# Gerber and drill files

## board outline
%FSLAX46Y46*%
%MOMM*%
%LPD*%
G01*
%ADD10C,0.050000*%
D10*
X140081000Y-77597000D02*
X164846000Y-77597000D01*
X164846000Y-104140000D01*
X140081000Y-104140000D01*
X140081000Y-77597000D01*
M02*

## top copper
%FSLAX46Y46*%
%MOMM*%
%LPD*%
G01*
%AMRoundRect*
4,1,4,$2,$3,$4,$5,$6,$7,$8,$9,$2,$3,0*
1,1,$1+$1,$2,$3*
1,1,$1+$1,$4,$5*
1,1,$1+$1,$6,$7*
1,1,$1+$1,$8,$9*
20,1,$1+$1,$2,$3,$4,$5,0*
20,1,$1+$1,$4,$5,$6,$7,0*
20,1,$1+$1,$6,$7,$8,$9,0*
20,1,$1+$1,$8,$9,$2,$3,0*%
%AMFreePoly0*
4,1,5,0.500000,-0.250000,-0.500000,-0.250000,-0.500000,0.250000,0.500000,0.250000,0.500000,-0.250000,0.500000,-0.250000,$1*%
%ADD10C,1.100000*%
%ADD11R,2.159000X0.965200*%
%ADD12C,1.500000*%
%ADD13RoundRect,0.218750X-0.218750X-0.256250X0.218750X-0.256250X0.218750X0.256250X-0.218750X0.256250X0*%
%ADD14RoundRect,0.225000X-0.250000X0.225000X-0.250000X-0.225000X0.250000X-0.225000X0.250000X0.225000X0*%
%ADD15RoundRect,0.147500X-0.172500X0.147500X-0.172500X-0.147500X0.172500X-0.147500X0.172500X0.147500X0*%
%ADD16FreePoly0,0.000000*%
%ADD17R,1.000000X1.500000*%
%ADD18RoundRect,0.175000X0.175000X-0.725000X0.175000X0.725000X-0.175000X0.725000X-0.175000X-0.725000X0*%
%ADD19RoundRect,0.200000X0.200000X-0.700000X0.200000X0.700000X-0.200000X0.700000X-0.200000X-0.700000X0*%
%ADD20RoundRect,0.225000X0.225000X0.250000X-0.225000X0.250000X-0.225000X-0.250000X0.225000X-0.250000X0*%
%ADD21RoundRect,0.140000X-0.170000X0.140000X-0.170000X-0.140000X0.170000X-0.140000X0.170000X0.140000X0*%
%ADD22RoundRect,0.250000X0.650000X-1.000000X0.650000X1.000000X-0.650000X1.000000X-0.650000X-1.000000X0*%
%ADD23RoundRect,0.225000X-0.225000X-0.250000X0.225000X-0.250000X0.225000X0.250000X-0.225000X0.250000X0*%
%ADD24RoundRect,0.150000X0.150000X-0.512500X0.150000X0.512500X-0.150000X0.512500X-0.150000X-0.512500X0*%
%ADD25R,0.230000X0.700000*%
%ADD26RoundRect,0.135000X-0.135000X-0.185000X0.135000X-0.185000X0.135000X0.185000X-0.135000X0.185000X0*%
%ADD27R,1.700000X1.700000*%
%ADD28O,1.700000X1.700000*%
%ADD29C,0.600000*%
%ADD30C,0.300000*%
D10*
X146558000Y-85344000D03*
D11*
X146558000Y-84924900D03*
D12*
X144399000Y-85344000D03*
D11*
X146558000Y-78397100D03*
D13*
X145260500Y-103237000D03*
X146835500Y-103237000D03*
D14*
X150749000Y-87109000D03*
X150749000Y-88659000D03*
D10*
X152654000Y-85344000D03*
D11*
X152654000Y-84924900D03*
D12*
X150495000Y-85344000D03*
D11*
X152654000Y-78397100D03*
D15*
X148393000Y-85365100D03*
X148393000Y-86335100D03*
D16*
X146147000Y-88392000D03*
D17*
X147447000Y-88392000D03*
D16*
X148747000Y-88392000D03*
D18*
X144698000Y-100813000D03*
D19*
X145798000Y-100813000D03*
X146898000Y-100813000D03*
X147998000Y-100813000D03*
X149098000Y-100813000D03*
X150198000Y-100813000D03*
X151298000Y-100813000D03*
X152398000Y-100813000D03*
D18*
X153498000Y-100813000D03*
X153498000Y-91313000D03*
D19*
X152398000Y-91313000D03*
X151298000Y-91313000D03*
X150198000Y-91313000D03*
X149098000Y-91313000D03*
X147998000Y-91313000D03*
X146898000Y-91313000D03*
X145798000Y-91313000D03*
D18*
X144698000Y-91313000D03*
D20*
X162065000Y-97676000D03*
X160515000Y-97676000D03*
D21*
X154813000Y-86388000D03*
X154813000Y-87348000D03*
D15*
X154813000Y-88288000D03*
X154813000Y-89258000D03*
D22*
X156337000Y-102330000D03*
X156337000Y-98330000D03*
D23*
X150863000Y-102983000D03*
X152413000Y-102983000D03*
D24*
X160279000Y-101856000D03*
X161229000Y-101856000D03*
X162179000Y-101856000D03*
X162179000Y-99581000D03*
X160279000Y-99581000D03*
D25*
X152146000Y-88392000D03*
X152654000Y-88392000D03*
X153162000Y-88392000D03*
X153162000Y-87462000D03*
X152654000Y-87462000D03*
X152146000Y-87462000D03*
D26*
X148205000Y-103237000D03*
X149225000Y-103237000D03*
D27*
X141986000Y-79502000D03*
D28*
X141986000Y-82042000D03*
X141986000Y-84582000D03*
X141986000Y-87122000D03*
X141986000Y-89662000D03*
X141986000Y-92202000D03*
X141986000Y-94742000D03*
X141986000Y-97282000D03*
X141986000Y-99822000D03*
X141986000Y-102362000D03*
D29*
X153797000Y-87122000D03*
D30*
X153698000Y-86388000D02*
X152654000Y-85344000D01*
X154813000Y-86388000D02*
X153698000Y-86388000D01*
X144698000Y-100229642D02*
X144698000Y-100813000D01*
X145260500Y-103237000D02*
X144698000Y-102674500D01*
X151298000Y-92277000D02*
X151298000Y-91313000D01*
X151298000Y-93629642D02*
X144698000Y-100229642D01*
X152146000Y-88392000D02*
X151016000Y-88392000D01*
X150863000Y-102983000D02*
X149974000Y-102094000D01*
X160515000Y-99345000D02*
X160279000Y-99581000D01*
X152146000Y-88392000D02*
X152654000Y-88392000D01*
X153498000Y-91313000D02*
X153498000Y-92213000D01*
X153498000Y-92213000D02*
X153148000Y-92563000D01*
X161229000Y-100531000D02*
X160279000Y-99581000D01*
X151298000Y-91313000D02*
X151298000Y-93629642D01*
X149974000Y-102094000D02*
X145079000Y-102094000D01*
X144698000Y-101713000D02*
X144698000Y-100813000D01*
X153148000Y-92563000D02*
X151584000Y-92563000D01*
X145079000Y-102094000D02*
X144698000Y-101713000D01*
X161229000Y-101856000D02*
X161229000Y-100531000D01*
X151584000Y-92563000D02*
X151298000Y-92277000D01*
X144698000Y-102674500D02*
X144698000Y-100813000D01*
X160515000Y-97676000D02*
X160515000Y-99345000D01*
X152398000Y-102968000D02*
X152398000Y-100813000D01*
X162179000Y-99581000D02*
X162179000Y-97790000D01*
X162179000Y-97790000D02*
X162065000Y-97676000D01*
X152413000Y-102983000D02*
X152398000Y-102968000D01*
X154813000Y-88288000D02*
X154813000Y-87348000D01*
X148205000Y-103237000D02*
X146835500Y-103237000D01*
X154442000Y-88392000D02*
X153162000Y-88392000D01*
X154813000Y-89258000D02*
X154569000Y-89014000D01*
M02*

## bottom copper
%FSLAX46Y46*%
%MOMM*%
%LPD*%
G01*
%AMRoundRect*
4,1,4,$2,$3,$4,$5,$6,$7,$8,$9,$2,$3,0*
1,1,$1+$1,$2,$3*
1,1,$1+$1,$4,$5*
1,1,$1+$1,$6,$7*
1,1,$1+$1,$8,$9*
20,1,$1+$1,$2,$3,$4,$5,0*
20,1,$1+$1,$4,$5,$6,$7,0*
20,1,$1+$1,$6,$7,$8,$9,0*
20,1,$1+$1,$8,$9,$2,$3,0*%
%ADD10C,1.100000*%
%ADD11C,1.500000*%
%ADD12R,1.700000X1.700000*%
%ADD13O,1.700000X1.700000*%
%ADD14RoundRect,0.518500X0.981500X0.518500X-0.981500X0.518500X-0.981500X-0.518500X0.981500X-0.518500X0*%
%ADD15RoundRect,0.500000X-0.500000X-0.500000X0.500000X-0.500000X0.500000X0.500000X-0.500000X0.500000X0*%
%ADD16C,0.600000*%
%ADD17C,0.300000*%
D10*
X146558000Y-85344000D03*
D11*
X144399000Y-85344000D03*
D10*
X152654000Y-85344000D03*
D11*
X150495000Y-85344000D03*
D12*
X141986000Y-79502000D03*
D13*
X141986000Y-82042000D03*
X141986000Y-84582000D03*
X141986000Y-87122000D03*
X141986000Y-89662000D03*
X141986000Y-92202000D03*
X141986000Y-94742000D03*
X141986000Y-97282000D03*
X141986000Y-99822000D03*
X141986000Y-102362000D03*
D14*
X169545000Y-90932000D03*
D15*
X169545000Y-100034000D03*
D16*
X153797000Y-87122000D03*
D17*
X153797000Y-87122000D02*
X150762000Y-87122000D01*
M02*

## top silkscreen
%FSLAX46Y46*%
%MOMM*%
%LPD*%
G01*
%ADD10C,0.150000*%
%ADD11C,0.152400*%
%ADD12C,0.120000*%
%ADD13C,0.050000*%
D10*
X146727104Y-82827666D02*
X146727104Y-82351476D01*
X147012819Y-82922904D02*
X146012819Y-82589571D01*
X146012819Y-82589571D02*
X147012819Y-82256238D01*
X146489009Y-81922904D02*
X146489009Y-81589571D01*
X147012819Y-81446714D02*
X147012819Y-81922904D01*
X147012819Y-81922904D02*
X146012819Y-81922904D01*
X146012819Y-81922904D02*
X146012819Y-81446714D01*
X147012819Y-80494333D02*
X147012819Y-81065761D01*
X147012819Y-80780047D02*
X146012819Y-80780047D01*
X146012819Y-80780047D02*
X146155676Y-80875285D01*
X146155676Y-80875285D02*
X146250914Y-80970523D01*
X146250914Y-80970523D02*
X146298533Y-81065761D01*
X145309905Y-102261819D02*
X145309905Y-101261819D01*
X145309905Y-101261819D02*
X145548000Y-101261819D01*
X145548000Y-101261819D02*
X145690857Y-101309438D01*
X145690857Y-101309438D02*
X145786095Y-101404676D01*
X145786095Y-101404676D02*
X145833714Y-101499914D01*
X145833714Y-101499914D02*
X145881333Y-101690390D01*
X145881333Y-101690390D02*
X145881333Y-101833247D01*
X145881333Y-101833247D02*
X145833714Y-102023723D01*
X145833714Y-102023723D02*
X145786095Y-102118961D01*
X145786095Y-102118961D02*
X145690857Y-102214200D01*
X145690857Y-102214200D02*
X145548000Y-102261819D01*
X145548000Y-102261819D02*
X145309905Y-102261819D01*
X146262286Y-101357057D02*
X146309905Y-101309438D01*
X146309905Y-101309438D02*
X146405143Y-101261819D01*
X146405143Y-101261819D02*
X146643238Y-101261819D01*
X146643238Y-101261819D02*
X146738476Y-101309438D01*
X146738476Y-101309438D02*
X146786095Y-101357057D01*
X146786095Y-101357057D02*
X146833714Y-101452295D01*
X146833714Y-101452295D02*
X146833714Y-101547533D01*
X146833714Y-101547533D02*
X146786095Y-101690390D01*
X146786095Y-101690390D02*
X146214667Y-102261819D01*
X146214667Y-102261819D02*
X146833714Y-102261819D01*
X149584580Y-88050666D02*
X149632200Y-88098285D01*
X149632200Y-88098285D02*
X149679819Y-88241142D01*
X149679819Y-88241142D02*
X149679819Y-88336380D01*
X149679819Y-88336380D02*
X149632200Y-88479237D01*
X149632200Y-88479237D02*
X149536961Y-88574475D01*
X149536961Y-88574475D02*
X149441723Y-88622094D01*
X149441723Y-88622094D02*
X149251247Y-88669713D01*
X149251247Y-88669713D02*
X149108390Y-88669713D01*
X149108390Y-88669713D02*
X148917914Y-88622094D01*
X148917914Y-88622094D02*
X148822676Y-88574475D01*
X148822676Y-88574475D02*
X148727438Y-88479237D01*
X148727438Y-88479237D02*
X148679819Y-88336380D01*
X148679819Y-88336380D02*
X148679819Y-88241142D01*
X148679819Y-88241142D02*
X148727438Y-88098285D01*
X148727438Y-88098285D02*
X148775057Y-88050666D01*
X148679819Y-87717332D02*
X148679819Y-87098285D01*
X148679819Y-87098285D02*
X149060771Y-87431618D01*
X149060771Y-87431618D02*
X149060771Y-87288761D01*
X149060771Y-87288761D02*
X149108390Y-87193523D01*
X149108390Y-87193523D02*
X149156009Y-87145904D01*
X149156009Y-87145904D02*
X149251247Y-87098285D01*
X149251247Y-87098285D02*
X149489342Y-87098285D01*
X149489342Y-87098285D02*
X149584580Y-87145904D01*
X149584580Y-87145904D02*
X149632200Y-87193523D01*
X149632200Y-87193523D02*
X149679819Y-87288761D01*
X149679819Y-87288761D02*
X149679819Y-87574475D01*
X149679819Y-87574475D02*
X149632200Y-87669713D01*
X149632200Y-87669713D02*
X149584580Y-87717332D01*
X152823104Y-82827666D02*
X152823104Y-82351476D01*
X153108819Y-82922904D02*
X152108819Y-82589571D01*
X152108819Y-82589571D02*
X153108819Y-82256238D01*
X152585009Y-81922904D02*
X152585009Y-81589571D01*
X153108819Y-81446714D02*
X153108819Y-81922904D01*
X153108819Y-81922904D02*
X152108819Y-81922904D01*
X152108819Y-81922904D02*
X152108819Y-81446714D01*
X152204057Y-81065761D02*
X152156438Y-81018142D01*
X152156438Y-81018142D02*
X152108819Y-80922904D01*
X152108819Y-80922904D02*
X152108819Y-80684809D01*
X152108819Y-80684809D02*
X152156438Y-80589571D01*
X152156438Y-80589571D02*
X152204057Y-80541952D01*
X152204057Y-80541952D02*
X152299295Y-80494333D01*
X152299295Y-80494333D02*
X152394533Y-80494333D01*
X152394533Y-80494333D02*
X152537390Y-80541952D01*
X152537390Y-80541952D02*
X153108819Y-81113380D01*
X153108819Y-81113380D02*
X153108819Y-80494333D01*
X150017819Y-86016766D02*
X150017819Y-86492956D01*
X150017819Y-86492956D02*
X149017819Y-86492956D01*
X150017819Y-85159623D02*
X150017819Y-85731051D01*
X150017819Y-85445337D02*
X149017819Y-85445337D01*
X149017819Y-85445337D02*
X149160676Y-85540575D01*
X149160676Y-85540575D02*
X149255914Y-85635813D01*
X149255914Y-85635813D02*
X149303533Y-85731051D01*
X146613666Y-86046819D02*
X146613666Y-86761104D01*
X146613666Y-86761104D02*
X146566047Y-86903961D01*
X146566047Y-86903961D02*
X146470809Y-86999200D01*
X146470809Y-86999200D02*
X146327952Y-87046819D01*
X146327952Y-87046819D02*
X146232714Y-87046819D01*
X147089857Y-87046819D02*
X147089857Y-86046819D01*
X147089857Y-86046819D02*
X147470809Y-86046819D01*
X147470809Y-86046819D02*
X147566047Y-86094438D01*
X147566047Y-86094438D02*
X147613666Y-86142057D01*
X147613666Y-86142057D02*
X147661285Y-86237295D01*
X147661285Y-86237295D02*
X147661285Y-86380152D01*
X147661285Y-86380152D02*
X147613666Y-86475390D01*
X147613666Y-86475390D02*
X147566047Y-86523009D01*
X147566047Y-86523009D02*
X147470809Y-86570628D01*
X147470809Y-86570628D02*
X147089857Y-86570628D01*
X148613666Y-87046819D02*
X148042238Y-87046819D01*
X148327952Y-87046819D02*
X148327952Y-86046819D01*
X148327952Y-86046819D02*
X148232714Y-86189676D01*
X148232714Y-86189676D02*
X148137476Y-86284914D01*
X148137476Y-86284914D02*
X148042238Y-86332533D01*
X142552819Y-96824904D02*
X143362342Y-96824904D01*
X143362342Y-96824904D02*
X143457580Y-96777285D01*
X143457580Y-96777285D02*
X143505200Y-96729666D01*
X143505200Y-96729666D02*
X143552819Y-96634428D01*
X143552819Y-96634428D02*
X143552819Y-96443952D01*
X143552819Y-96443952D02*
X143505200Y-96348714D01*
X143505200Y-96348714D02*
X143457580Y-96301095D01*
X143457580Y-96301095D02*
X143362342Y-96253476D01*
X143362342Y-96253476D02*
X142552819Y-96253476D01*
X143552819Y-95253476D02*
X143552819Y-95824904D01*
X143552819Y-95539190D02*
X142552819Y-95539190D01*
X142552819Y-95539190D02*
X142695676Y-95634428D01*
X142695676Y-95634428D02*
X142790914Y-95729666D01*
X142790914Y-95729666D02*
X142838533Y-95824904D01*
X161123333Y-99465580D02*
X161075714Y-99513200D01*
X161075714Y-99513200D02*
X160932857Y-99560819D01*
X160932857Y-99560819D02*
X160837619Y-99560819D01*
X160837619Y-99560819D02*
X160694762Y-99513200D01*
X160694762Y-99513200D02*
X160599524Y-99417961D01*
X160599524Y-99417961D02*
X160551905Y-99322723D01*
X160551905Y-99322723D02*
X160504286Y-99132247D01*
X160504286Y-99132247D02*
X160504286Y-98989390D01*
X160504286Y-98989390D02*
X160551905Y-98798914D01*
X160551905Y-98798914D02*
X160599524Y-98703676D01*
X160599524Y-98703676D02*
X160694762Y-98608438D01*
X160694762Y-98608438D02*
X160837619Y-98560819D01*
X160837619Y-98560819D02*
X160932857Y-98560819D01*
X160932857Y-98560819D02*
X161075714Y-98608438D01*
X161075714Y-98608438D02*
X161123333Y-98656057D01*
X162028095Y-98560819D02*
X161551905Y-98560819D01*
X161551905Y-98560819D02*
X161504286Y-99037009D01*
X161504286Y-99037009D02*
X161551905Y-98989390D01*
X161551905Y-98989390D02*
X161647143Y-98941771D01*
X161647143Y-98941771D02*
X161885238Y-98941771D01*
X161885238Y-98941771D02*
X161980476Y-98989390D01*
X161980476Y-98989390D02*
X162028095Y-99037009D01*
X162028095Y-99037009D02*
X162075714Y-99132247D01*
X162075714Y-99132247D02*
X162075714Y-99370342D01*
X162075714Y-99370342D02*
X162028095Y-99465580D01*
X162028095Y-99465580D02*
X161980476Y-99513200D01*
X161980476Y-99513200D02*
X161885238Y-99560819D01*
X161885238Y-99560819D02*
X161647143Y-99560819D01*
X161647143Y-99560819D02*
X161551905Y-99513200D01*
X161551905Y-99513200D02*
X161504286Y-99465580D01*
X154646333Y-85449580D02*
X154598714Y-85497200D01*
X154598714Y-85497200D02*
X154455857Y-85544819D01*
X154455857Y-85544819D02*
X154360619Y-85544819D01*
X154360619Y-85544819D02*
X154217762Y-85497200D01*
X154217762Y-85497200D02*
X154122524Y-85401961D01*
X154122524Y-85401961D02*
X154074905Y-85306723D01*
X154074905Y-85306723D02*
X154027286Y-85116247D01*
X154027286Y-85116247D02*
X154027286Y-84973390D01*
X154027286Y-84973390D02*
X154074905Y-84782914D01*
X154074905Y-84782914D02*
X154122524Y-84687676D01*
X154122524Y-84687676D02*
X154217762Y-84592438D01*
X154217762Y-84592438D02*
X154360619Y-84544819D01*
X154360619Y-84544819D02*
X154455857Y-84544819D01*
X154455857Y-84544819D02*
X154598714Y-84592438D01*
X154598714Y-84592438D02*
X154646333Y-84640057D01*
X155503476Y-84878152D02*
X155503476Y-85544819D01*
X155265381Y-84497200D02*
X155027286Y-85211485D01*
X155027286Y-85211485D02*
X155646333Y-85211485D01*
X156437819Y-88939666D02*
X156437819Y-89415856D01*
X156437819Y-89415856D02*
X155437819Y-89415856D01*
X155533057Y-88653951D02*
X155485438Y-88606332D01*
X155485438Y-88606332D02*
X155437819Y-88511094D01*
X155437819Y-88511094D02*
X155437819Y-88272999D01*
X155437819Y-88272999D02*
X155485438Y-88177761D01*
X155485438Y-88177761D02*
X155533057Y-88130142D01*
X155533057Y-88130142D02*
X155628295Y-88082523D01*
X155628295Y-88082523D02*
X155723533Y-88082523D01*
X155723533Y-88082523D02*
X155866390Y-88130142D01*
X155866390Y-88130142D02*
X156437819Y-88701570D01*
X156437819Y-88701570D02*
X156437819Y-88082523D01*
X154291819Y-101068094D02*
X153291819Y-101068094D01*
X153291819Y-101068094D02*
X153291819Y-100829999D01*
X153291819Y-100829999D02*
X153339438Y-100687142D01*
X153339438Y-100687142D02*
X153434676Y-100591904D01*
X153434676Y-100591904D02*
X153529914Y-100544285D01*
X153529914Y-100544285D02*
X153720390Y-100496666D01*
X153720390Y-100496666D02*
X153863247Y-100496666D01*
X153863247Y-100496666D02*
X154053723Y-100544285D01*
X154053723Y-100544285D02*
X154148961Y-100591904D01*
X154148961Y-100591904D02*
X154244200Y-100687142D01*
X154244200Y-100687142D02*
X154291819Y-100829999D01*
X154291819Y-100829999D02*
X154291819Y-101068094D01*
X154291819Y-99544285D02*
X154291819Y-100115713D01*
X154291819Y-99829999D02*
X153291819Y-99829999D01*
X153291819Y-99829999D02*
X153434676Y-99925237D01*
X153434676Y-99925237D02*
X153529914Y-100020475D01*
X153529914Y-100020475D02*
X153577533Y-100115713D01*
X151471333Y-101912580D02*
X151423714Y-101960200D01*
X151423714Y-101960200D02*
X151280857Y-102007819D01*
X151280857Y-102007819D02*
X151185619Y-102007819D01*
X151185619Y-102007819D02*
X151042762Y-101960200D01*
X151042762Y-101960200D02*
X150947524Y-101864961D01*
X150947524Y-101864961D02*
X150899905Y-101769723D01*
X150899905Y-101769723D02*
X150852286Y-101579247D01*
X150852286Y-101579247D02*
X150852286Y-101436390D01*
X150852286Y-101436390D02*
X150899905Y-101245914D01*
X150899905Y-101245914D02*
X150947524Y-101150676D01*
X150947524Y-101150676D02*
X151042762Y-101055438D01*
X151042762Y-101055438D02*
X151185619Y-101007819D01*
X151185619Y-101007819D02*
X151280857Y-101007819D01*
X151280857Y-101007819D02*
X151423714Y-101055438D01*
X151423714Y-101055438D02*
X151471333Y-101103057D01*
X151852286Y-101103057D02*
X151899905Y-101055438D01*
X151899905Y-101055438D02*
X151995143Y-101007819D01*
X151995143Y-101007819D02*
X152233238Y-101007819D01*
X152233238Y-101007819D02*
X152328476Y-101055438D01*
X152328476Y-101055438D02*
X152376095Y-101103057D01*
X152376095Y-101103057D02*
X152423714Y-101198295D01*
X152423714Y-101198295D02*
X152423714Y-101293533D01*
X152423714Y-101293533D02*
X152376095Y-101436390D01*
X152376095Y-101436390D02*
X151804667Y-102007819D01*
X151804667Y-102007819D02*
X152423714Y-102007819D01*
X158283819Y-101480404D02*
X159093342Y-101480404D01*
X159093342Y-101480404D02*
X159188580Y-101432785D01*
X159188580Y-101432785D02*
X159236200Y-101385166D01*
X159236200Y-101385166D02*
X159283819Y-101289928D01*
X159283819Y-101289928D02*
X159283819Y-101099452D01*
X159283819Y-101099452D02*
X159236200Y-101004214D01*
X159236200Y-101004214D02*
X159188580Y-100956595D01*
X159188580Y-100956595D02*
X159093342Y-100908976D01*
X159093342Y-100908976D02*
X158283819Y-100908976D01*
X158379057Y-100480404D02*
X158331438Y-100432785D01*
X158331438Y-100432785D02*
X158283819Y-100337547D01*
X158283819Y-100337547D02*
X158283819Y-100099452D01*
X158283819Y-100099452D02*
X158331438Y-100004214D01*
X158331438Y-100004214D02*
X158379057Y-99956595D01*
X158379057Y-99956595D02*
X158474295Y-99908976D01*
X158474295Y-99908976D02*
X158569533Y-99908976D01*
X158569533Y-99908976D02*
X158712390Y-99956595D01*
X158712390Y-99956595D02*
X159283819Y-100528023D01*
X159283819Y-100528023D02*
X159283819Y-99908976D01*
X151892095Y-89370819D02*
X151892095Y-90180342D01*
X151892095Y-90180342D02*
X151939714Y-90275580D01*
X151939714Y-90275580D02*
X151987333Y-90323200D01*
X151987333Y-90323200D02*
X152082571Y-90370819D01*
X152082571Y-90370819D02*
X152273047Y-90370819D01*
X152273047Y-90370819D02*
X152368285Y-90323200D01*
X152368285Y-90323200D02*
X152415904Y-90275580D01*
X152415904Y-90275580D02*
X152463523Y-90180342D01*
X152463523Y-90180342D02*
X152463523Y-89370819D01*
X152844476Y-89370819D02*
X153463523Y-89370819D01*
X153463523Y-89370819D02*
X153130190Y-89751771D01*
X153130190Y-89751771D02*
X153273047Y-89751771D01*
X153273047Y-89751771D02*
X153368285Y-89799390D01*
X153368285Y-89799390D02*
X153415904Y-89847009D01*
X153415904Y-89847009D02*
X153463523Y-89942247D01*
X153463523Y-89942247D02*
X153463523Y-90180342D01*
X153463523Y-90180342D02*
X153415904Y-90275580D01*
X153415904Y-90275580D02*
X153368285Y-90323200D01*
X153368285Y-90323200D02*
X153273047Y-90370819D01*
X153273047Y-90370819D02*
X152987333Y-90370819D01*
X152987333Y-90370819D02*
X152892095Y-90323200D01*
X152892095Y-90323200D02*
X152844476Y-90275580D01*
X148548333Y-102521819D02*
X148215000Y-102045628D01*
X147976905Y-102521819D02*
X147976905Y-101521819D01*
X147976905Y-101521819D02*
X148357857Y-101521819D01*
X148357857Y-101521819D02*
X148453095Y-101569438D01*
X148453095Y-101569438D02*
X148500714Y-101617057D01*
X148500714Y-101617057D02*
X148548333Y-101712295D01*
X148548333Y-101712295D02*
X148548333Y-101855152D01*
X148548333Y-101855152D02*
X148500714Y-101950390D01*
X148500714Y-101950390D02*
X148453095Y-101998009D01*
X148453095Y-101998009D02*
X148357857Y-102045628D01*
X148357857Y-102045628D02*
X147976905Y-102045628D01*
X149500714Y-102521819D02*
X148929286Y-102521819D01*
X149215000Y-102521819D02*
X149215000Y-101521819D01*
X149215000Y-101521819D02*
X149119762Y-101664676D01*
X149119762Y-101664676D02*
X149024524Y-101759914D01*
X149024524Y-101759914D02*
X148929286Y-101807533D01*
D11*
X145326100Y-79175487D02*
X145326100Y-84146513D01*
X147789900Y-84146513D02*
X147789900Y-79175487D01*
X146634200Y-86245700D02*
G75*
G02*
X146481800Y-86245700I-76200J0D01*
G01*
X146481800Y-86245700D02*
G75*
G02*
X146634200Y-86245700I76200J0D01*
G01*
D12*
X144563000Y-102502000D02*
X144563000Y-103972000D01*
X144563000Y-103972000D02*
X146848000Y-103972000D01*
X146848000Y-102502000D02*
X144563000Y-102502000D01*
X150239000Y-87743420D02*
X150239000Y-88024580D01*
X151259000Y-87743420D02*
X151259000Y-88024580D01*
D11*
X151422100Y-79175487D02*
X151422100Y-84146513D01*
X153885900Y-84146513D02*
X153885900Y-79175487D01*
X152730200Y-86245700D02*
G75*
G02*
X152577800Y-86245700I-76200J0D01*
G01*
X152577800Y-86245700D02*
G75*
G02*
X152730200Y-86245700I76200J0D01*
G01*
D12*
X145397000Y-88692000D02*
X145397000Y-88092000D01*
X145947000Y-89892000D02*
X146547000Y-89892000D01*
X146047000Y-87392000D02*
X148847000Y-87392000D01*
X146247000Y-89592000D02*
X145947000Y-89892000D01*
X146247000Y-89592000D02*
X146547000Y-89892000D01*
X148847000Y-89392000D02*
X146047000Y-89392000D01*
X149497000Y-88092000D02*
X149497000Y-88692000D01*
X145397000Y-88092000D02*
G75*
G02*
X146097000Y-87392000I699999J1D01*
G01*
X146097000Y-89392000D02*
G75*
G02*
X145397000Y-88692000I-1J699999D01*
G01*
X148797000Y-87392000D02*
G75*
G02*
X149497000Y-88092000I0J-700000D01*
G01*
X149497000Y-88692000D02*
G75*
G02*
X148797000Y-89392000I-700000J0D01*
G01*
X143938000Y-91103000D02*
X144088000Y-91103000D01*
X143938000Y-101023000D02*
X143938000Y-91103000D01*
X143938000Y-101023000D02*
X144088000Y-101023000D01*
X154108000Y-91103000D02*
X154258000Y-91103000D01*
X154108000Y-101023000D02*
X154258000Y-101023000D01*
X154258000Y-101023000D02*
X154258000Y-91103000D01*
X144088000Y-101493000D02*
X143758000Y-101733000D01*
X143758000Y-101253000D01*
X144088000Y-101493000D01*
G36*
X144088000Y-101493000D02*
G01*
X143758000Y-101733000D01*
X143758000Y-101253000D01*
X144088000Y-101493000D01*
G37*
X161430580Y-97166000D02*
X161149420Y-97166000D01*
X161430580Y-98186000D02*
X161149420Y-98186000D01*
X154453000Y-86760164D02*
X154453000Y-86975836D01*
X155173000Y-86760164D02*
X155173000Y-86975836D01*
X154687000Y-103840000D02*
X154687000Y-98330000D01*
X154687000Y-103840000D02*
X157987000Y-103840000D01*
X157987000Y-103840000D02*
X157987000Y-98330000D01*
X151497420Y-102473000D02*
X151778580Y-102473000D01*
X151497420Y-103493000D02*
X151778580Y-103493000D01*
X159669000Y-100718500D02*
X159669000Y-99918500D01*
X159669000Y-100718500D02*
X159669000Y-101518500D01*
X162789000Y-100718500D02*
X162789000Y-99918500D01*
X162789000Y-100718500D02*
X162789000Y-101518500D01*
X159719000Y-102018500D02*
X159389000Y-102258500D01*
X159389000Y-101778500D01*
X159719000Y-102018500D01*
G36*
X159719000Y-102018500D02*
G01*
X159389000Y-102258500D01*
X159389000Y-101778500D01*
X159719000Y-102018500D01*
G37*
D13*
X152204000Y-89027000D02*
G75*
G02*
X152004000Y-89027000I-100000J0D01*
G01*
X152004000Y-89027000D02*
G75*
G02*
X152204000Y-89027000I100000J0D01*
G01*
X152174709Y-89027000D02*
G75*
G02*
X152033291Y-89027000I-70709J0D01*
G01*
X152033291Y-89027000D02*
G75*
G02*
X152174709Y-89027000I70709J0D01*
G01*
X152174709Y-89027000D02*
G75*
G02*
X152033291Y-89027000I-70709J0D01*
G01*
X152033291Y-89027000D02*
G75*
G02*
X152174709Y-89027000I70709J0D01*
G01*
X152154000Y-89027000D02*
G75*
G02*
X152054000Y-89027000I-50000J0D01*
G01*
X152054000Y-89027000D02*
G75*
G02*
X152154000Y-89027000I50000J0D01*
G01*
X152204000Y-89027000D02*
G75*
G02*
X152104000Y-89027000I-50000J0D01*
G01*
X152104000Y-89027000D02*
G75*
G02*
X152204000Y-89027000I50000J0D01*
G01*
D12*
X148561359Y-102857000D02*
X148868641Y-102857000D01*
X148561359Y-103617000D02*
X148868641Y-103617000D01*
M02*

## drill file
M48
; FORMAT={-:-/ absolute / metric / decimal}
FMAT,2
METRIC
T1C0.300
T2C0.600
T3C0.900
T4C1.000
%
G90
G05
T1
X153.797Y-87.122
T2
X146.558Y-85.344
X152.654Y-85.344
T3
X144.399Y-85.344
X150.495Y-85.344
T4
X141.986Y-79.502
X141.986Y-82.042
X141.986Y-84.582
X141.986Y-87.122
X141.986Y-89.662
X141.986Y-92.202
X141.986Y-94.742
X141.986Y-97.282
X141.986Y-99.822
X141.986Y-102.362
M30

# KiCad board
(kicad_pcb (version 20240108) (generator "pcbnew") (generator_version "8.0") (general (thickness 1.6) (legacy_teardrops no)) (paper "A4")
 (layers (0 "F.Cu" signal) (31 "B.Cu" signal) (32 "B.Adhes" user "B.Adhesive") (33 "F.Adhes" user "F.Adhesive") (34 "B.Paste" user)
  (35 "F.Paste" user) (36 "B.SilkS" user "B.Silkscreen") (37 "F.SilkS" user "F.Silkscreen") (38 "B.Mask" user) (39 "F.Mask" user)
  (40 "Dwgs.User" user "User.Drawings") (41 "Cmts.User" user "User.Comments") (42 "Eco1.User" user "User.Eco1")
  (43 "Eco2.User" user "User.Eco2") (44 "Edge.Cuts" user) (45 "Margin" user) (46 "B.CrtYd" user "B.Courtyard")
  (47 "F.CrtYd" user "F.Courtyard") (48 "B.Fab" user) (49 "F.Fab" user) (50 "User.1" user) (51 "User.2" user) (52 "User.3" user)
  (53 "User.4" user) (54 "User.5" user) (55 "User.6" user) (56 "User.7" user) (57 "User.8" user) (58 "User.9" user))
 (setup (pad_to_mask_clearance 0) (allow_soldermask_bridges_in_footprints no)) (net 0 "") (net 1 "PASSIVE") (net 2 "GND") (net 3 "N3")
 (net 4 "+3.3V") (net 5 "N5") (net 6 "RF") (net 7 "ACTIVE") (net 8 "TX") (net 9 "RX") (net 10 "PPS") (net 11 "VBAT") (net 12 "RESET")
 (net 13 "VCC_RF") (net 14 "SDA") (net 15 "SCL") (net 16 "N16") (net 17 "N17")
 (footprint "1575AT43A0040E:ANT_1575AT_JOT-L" (layer "F.Cu") (at 146.558 81.661 90)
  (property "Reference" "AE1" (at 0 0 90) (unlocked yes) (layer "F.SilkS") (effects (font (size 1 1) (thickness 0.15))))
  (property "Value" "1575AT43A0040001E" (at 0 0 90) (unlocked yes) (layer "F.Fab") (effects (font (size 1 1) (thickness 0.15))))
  (fp_line (start 2.485513 -1.2319) (end -2.485513 -1.2319) (stroke (width 0.1524) (type solid)) (layer "F.SilkS"))
  (fp_line (start -2.485513 1.2319) (end 2.485513 1.2319) (stroke (width 0.1524) (type solid)) (layer "F.SilkS"))
  (fp_circle (center -4.5847 0) (end -4.5085 0) (stroke (width 0.1524) (type solid)) (fill none) (layer "F.SilkS"))
  (pad "1" thru_hole circle (at -3.683 0 90) (size 1.1 1.1) (drill 0.6) (layers "*.Cu" "*.Mask") (remove_unused_layers no) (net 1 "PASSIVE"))
  (pad "1" smd rect (at -3.2639 0 90) (size 0.9652 2.159) (layers "F.Cu" "F.Paste" "F.Mask") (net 1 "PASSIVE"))
  (pad "2" thru_hole circle (at -3.683 -2.159 90) (size 1.5 1.5) (drill 0.9) (layers "*.Cu" "*.Mask") (remove_unused_layers no)
   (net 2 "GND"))
  (pad "3" smd rect (at 3.2639 0 90) (size 0.9652 2.159) (layers "F.Cu" "F.Paste" "F.Mask"))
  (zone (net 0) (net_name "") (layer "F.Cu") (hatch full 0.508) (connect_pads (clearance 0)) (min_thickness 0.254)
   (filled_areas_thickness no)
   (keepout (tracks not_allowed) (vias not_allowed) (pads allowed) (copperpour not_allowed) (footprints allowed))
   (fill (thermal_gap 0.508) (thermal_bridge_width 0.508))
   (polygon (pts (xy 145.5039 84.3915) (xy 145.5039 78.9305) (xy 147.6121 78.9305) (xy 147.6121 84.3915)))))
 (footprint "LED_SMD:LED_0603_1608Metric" (layer "F.Cu") (at 146.048 103.237)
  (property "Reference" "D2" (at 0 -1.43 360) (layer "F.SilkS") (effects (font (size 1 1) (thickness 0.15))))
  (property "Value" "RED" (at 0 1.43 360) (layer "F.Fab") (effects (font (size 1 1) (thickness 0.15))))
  (fp_line (start -1.485 -0.735) (end -1.485 0.735) (stroke (width 0.12) (type solid)) (layer "F.SilkS"))
  (fp_line (start -1.485 0.735) (end 0.8 0.735) (stroke (width 0.12) (type solid)) (layer "F.SilkS"))
  (fp_line (start 0.8 -0.735) (end -1.485 -0.735) (stroke (width 0.12) (type solid)) (layer "F.SilkS"))
  (pad "1" smd roundrect (at -0.7875 0) (size 0.875 0.95) (layers "F.Cu" "F.Paste" "F.Mask") (roundrect_rratio 0.25) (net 2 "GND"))
  (pad "2" smd roundrect (at 0.7875 0) (size 0.875 0.95) (layers "F.Cu" "F.Paste" "F.Mask") (roundrect_rratio 0.25) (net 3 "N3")))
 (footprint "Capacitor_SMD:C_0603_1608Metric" (layer "F.Cu") (at 150.749 87.884 -90)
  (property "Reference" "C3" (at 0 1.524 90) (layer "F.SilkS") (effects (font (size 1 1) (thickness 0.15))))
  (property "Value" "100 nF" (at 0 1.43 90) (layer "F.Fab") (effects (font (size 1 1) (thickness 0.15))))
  (fp_line (start -0.14058 0.51) (end 0.14058 0.51) (stroke (width 0.12) (type solid)) (layer "F.SilkS"))
  (fp_line (start -0.14058 -0.51) (end 0.14058 -0.51) (stroke (width 0.12) (type solid)) (layer "F.SilkS"))
  (pad "1" smd roundrect (at -0.775 0 270) (size 0.9 0.95) (layers "F.Cu" "F.Paste" "F.Mask") (roundrect_rratio 0.25) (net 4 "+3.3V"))
  (pad "2" smd roundrect (at 0.775 0 270) (size 0.9 0.95) (layers "F.Cu" "F.Paste" "F.Mask") (roundrect_rratio 0.25) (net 2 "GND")))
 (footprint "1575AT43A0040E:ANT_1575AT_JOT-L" (layer "F.Cu") (at 152.654 81.661 90)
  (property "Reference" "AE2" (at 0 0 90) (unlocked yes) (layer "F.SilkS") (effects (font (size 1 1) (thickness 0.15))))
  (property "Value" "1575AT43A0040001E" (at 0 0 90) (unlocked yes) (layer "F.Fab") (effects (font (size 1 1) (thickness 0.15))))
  (fp_line (start 2.485513 -1.2319) (end -2.485513 -1.2319) (stroke (width 0.1524) (type solid)) (layer "F.SilkS"))
  (fp_line (start -2.485513 1.2319) (end 2.485513 1.2319) (stroke (width 0.1524) (type solid)) (layer "F.SilkS"))
  (fp_circle (center -4.5847 0) (end -4.5085 0) (stroke (width 0.1524) (type solid)) (fill none) (layer "F.SilkS"))
  (pad "1" thru_hole circle (at -3.683 0 90) (size 1.1 1.1) (drill 0.6) (layers "*.Cu" "*.Mask") (remove_unused_layers no) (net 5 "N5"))
  (pad "1" smd rect (at -3.2639 0 90) (size 0.9652 2.159) (layers "F.Cu" "F.Paste" "F.Mask") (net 5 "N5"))
  (pad "2" thru_hole circle (at -3.683 -2.159 90) (size 1.5 1.5) (drill 0.9) (layers "*.Cu" "*.Mask") (remove_unused_layers no)
   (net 2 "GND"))
  (pad "3" smd rect (at 3.2639 0 90) (size 0.9652 2.159) (layers "F.Cu" "F.Paste" "F.Mask"))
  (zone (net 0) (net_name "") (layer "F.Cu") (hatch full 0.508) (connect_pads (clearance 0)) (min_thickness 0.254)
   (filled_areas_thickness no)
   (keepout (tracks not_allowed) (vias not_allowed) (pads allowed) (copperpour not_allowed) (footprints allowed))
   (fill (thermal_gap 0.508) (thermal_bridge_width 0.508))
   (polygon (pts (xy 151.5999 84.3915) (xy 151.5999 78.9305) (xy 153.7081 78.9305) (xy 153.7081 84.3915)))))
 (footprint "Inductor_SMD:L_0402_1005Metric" (layer "F.Cu") (at 148.393 85.8501 -90)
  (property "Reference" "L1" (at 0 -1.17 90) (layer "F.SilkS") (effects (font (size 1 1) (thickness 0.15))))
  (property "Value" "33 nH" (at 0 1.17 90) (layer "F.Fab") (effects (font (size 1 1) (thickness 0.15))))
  (pad "1" smd roundrect (at -0.485 0 270) (size 0.59 0.64) (layers "F.Cu" "F.Paste" "F.Mask") (roundrect_rratio 0.25) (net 1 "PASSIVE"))
  (pad "2" smd roundrect (at 0.485 0 270) (size 0.59 0.64) (layers "F.Cu" "F.Paste" "F.Mask") (roundrect_rratio 0.25) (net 2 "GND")))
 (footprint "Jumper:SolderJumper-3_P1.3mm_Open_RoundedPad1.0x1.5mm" (layer "F.Cu") (at 147.447 88.392)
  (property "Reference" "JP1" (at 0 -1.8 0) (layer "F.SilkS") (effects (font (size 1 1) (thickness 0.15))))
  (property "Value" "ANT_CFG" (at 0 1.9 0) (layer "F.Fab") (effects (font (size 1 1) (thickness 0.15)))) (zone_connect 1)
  (fp_line (start -2.05 0.3) (end -2.05 -0.3) (stroke (width 0.12) (type solid)) (layer "F.SilkS"))
  (fp_line (start -1.5 1.5) (end -0.9 1.5) (stroke (width 0.12) (type solid)) (layer "F.SilkS"))
  (fp_line (start -1.4 -1) (end 1.4 -1) (stroke (width 0.12) (type solid)) (layer "F.SilkS"))
  (fp_line (start -1.2 1.2) (end -1.5 1.5) (stroke (width 0.12) (type solid)) (layer "F.SilkS"))
  (fp_line (start -1.2 1.2) (end -0.9 1.5) (stroke (width 0.12) (type solid)) (layer "F.SilkS"))
  (fp_line (start 1.4 1) (end -1.4 1) (stroke (width 0.12) (type solid)) (layer "F.SilkS"))
  (fp_line (start 2.05 -0.3) (end 2.05 0.3) (stroke (width 0.12) (type solid)) (layer "F.SilkS"))
  (fp_arc (start -2.05 -0.3) (mid -1.844975 -0.794975) (end -1.35 -1) (stroke (width 0.12) (type solid)) (layer "F.SilkS"))
  (fp_arc (start -1.35 1) (mid -1.844975 0.794975) (end -2.05 0.3) (stroke (width 0.12) (type solid)) (layer "F.SilkS"))
  (fp_arc (start 1.35 -1) (mid 1.844975 -0.794975) (end 2.05 -0.3) (stroke (width 0.12) (type solid)) (layer "F.SilkS"))
  (fp_arc (start 2.05 0.3) (mid 1.844975 0.794975) (end 1.35 1) (stroke (width 0.12) (type solid)) (layer "F.SilkS"))
  (pad "1" smd custom (at -1.3 0) (size 1 0.5) (layers "F.Cu" "F.Mask") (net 1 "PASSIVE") (zone_connect 2) (thermal_bridge_angle 45)
   (options (clearance outline) (anchor rect)) (primitives))
  (pad "2" smd rect (at 0 0) (size 1 1.5) (layers "F.Cu" "F.Mask") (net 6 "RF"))
  (pad "3" smd custom (at 1.3 0) (size 1 0.5) (layers "F.Cu" "F.Mask") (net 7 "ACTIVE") (zone_connect 2) (thermal_bridge_angle 45)
   (options (clearance outline) (anchor rect)) (primitives)))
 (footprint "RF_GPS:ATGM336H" (layer "F.Cu") (at 149.098 96.063 90)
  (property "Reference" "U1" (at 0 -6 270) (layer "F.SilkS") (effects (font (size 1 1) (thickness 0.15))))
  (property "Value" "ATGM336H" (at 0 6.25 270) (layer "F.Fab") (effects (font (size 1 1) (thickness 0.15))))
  (fp_line (start 4.96 -5.16) (end 4.96 -5.01) (stroke (width 0.12) (type solid)) (layer "F.SilkS"))
  (fp_line (start -4.96 -5.16) (end 4.96 -5.16) (stroke (width 0.12) (type solid)) (layer "F.SilkS"))
  (fp_line (start -4.96 -5.16) (end -4.96 -5.01) (stroke (width 0.12) (type solid)) (layer "F.SilkS"))
  (fp_line (start 4.96 5.01) (end 4.96 5.16) (stroke (width 0.12) (type solid)) (layer "F.SilkS"))
  (fp_line (start -4.96 5.01) (end -4.96 5.16) (stroke (width 0.12) (type solid)) (layer "F.SilkS"))
  (fp_line (start -4.96 5.16) (end 4.96 5.16) (stroke (width 0.12) (type solid)) (layer "F.SilkS"))
  (fp_poly
   (pts (xy -5.43 -5.01) (xy -5.67 -5.34) (xy -5.19 -5.34) (xy -5.43 -5.01)) (stroke (width 0.12) (type solid)) (fill solid)
   (layer "F.SilkS"))
  (pad "1" smd roundrect (at -4.75 -4.4 90) (size 1.8 0.7) (layers "F.Cu" "F.Paste" "F.Mask") (roundrect_rratio 0.25) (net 2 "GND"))
  (pad "2" smd roundrect (at -4.75 -3.3 90) (size 1.8 0.8) (layers "F.Cu" "F.Paste" "F.Mask") (roundrect_rratio 0.25) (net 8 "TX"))
  (pad "3" smd roundrect (at -4.75 -2.2 90) (size 1.8 0.8) (layers "F.Cu" "F.Paste" "F.Mask") (roundrect_rratio 0.25) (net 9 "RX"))
  (pad "4" smd roundrect (at -4.75 -1.1 90) (size 1.8 0.8) (layers "F.Cu" "F.Paste" "F.Mask") (roundrect_rratio 0.25) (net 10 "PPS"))
  (pad "5" smd roundrect (at -4.75 0 90) (size 1.8 0.8) (layers "F.Cu" "F.Paste" "F.Mask") (roundrect_rratio 0.25) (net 4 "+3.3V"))
  (pad "6" smd roundrect (at -4.75 1.1 90) (size 1.8 0.8) (layers "F.Cu" "F.Paste" "F.Mask") (roundrect_rratio 0.25) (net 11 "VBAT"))
  (pad "7" smd roundrect (at -4.75 2.2 90) (size 1.8 0.8) (layers "F.Cu" "F.Paste" "F.Mask") (roundrect_rratio 0.25))
  (pad "8" smd roundrect (at -4.75 3.3 90) (size 1.8 0.8) (layers "F.Cu" "F.Paste" "F.Mask") (roundrect_rratio 0.25) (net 4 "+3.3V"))
  (pad "9" smd roundrect (at -4.75 4.4 90) (size 1.8 0.7) (layers "F.Cu" "F.Paste" "F.Mask") (roundrect_rratio 0.25) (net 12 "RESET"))
  (pad "10" smd roundrect (at 4.75 4.4 90) (size 1.8 0.7) (layers "F.Cu" "F.Paste" "F.Mask") (roundrect_rratio 0.25) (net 2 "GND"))
  (pad "11" smd roundrect (at 4.75 3.3 90) (size 1.8 0.8) (layers "F.Cu" "F.Paste" "F.Mask") (roundrect_rratio 0.25) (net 6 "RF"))
  (pad "12" smd roundrect (at 4.75 2.2 90) (size 1.8 0.8) (layers "F.Cu" "F.Paste" "F.Mask") (roundrect_rratio 0.25) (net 2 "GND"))
  (pad "13" smd roundrect (at 4.75 1.1 90) (size 1.8 0.8) (layers "F.Cu" "F.Paste" "F.Mask") (roundrect_rratio 0.25))
  (pad "14" smd roundrect (at 4.75 0 90) (size 1.8 0.8) (layers "F.Cu" "F.Paste" "F.Mask") (roundrect_rratio 0.25) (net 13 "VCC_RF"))
  (pad "15" smd roundrect (at 4.75 -1.1 90) (size 1.8 0.8) (layers "F.Cu" "F.Paste" "F.Mask") (roundrect_rratio 0.25))
  (pad "16" smd roundrect (at 4.75 -2.2 90) (size 1.8 0.8) (layers "F.Cu" "F.Paste" "F.Mask") (roundrect_rratio 0.25) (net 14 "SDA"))
  (pad "17" smd roundrect (at 4.75 -3.3 90) (size 1.8 0.8) (layers "F.Cu" "F.Paste" "F.Mask") (roundrect_rratio 0.25) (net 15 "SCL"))
  (pad "18" smd roundrect (at 4.75 -4.4 90) (size 1.8 0.7) (layers "F.Cu" "F.Paste" "F.Mask") (roundrect_rratio 0.25)))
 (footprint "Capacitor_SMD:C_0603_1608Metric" (layer "F.Cu") (at 161.29 97.676 180)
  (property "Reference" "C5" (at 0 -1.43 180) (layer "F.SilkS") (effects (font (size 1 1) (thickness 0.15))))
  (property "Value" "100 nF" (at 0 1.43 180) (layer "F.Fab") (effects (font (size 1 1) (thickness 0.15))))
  (fp_line (start -0.14058 0.51) (end 0.14058 0.51) (stroke (width 0.12) (type solid)) (layer "F.SilkS"))
  (fp_line (start -0.14058 -0.51) (end 0.14058 -0.51) (stroke (width 0.12) (type solid)) (layer "F.SilkS"))
  (pad "1" smd roundrect (at -0.775 0 180) (size 0.9 0.95) (layers "F.Cu" "F.Paste" "F.Mask") (roundrect_rratio 0.25) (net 4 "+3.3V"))
  (pad "2" smd roundrect (at 0.775 0 180) (size 0.9 0.95) (layers "F.Cu" "F.Paste" "F.Mask") (roundrect_rratio 0.25) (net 2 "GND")))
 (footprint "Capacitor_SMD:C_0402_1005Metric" (layer "F.Cu") (at 154.813 86.868 -90)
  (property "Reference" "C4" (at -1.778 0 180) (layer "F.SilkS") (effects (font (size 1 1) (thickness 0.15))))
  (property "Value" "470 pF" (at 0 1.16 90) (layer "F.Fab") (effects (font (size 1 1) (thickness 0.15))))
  (fp_line (start -0.107836 0.36) (end 0.107836 0.36) (stroke (width 0.12) (type solid)) (layer "F.SilkS"))
  (fp_line (start -0.107836 -0.36) (end 0.107836 -0.36) (stroke (width 0.12) (type solid)) (layer "F.SilkS"))
  (pad "1" smd roundrect (at -0.48 0 270) (size 0.56 0.62) (layers "F.Cu" "F.Paste" "F.Mask") (roundrect_rratio 0.25) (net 5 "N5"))
  (pad "2" smd roundrect (at 0.48 0 270) (size 0.56 0.62) (layers "F.Cu" "F.Paste" "F.Mask") (roundrect_rratio 0.25) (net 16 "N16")))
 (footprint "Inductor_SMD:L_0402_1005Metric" (layer "F.Cu") (at 154.813 88.773 -90)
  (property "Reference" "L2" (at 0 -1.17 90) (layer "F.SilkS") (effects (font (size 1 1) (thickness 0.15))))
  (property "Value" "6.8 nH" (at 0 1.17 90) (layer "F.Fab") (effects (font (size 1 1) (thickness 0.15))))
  (pad "1" smd roundrect (at -0.485 0 270) (size 0.59 0.64) (layers "F.Cu" "F.Paste" "F.Mask") (roundrect_rratio 0.25) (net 16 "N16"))
  (pad "2" smd roundrect (at 0.485 0 270) (size 0.59 0.64) (layers "F.Cu" "F.Paste" "F.Mask") (roundrect_rratio 0.25) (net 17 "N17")))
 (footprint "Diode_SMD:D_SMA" (layer "F.Cu") (at 156.337 100.33 90)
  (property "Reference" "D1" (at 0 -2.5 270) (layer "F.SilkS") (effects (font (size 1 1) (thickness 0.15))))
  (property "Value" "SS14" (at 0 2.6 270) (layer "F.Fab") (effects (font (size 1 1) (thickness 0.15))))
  (fp_line (start -3.51 -1.65) (end 2 -1.65) (stroke (width 0.12) (type solid)) (layer "F.SilkS"))
  (fp_line (start -3.51 -1.65) (end -3.51 1.65) (stroke (width 0.12) (type solid)) (layer "F.SilkS"))
  (fp_line (start -3.51 1.65) (end 2 1.65) (stroke (width 0.12) (type solid)) (layer "F.SilkS"))
  (pad "1" smd roundrect (at -2 0 90) (size 2.5 1.8) (layers "F.Cu" "F.Paste" "F.Mask") (roundrect_rratio 0.1388888889) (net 11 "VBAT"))
  (pad "2" smd roundrect (at 2 0 90) (size 2.5 1.8) (layers "F.Cu" "F.Paste" "F.Mask") (roundrect_rratio 0.1388888889) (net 4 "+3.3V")))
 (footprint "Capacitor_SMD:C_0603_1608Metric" (layer "F.Cu") (at 151.638 102.983)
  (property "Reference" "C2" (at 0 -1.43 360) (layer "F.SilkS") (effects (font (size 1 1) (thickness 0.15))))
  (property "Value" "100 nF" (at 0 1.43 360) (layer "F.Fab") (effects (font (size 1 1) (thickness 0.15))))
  (fp_line (start -0.14058 -0.51) (end 0.14058 -0.51) (stroke (width 0.12) (type solid)) (layer "F.SilkS"))
  (fp_line (start -0.14058 0.51) (end 0.14058 0.51) (stroke (width 0.12) (type solid)) (layer "F.SilkS"))
  (pad "1" smd roundrect (at -0.775 0) (size 0.9 0.95) (layers "F.Cu" "F.Paste" "F.Mask") (roundrect_rratio 0.25) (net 2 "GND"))
  (pad "2" smd roundrect (at 0.775 0) (size 0.9 0.95) (layers "F.Cu" "F.Paste" "F.Mask") (roundrect_rratio 0.25) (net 4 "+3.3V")))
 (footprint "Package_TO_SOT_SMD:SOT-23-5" (layer "F.Cu") (at 161.229 100.7185 90)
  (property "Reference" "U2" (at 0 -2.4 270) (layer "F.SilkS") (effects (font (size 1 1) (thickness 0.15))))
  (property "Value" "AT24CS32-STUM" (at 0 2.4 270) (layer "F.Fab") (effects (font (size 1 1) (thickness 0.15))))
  (fp_line (start 0 -1.56) (end 0.8 -1.56) (stroke (width 0.12) (type solid)) (layer "F.SilkS"))
  (fp_line (start 0 -1.56) (end -0.8 -1.56) (stroke (width 0.12) (type solid)) (layer "F.SilkS"))
  (fp_line (start 0 1.56) (end 0.8 1.56) (stroke (width 0.12) (type solid)) (layer "F.SilkS"))
  (fp_line (start 0 1.56) (end -0.8 1.56) (stroke (width 0.12) (type solid)) (layer "F.SilkS"))
  (fp_poly
   (pts (xy -1.3 -1.51) (xy -1.54 -1.84) (xy -1.06 -1.84) (xy -1.3 -1.51)) (stroke (width 0.12) (type solid)) (fill solid) (layer "F.SilkS"))
  (pad "1" smd roundrect (at -1.1375 -0.95 90) (size 1.325 0.6) (layers "F.Cu" "F.Paste" "F.Mask") (roundrect_rratio 0.25) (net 15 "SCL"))
  (pad "2" smd roundrect (at -1.1375 0 90) (size 1.325 0.6) (layers "F.Cu" "F.Paste" "F.Mask") (roundrect_rratio 0.25) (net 2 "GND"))
  (pad "3" smd roundrect (at -1.1375 0.95 90) (size 1.325 0.6) (layers "F.Cu" "F.Paste" "F.Mask") (roundrect_rratio 0.25) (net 14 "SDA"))
  (pad "4" smd roundrect (at 1.1375 0.95 90) (size 1.325 0.6) (layers "F.Cu" "F.Paste" "F.Mask") (roundrect_rratio 0.25) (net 4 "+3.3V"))
  (pad "5" smd roundrect (at 1.1375 -0.95 90) (size 1.325 0.6) (layers "F.Cu" "F.Paste" "F.Mask") (roundrect_rratio 0.25) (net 2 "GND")))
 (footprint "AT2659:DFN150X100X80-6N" (layer "F.Cu") (at 152.654 87.927 90)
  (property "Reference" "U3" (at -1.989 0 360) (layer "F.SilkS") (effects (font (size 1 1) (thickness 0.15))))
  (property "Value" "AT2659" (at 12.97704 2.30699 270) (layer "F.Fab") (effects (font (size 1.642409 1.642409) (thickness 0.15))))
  (fp_circle (center -1.1 -0.55) (end -1 -0.55) (stroke (width 0.05) (type solid)) (fill none) (layer "F.SilkS"))
  (fp_circle (center -1.1 -0.55) (end -1.029291 -0.55) (stroke (width 0.05) (type solid)) (fill none) (layer "F.SilkS"))
  (fp_circle (center -1.1 -0.55) (end -1.029291 -0.55) (stroke (width 0.05) (type solid)) (fill none) (layer "F.SilkS"))
  (fp_circle (center -1.1 -0.55) (end -1.05 -0.55) (stroke (width 0.05) (type solid)) (fill none) (layer "F.SilkS"))
  (fp_circle (center -1.1 -0.5) (end -1.05 -0.5) (stroke (width 0.05) (type solid)) (fill none) (layer "F.SilkS"))
  (pad "1" smd rect (at -0.465 -0.508 90) (size 0.7 0.23) (layers "F.Cu" "F.Paste" "F.Mask") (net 2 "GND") (solder_mask_margin 0.102))
  (pad "2" smd rect (at -0.465 0 90) (size 0.7 0.23) (layers "F.Cu" "F.Paste" "F.Mask") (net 2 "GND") (solder_mask_margin 0.102))
  (pad "3" smd rect (at -0.465 0.508 90) (size 0.7 0.23) (layers "F.Cu" "F.Paste" "F.Mask") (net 17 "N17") (solder_mask_margin 0.102))
  (pad "4" smd rect (at 0.465 0.508 90) (size 0.7 0.23) (layers "F.Cu" "F.Paste" "F.Mask") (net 4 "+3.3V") (solder_mask_margin 0.102))
  (pad "5" smd rect (at 0.465 0 90) (size 0.7 0.23) (layers "F.Cu" "F.Paste" "F.Mask") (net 4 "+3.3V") (solder_mask_margin 0.102))
  (pad "6" smd rect (at 0.465 -0.508 90) (size 0.7 0.23) (layers "F.Cu" "F.Paste" "F.Mask") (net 7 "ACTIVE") (solder_mask_margin 0.102)))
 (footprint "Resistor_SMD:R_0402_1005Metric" (layer "F.Cu") (at 148.715 103.237)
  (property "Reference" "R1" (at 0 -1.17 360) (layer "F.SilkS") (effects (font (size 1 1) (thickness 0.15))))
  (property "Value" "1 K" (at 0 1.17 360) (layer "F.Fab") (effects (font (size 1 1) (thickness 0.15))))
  (fp_line (start -0.153641 -0.38) (end 0.153641 -0.38) (stroke (width 0.12) (type solid)) (layer "F.SilkS"))
  (fp_line (start -0.153641 0.38) (end 0.153641 0.38) (stroke (width 0.12) (type solid)) (layer "F.SilkS"))
  (pad "1" smd roundrect (at -0.51 0) (size 0.54 0.64) (layers "F.Cu" "F.Paste" "F.Mask") (roundrect_rratio 0.25) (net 3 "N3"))
  (pad "2" smd roundrect (at 0.51 0) (size 0.54 0.64) (layers "F.Cu" "F.Paste" "F.Mask") (roundrect_rratio 0.25) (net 10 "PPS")))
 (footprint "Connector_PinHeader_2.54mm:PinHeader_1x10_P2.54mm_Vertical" (layer "B.Cu") (at 141.986 79.502 180)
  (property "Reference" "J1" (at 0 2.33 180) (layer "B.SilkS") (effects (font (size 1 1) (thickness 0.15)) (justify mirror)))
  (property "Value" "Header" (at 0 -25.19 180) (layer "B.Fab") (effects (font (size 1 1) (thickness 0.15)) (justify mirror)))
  (pad "1" thru_hole rect (at 0 0 180) (size 1.7 1.7) (drill 1) (layers "*.Cu" "*.Mask") (remove_unused_layers no) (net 2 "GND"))
  (pad "2" thru_hole oval (at 0 -2.54 180) (size 1.7 1.7) (drill 1) (layers "*.Cu" "*.Mask") (remove_unused_layers no) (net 4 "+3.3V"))
  (pad "3" thru_hole oval (at 0 -5.08 180) (size 1.7 1.7) (drill 1) (layers "*.Cu" "*.Mask") (remove_unused_layers no) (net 11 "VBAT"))
  (pad "4" thru_hole oval (at 0 -7.62 180) (size 1.7 1.7) (drill 1) (layers "*.Cu" "*.Mask") (remove_unused_layers no) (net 13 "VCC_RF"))
  (pad "5" thru_hole oval (at 0 -10.16 180) (size 1.7 1.7) (drill 1) (layers "*.Cu" "*.Mask") (remove_unused_layers no) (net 12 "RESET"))
  (pad "6" thru_hole oval (at 0 -12.7 180) (size 1.7 1.7) (drill 1) (layers "*.Cu" "*.Mask") (remove_unused_layers no) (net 10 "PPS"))
  (pad "7" thru_hole oval (at 0 -15.24 180) (size 1.7 1.7) (drill 1) (layers "*.Cu" "*.Mask") (remove_unused_layers no) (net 15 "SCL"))
  (pad "8" thru_hole oval (at 0 -17.78 180) (size 1.7 1.7) (drill 1) (layers "*.Cu" "*.Mask") (remove_unused_layers no) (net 14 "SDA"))
  (pad "9" thru_hole oval (at 0 -20.32 180) (size 1.7 1.7) (drill 1) (layers "*.Cu" "*.Mask") (remove_unused_layers no) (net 8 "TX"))
  (pad "10" thru_hole oval (at 0 -22.86 180) (size 1.7 1.7) (drill 1) (layers "*.Cu" "*.Mask") (remove_unused_layers no) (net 9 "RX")))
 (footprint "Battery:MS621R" (layer "B.Cu") (at 169.545 100.055 90)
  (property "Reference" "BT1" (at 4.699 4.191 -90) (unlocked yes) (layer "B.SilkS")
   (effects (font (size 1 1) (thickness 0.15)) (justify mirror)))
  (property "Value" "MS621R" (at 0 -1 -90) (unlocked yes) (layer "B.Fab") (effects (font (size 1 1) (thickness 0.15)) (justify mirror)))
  (pad "1" smd roundrect (at 9.123 0 180) (size 3 2.074) (layers "B.Cu" "B.Paste" "B.Mask") (roundrect_rratio 0.25) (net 11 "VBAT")
   (thermal_bridge_angle 45))
  (pad "2" smd roundrect (at 0.021 0) (size 2 2) (layers "B.Cu" "B.Paste" "B.Mask") (roundrect_rratio 0.25) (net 2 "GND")
   (thermal_bridge_angle 45)))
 (gr_rect (start 140.081 77.597) (end 164.846 104.14) (stroke (width 0.05) (type default)) (fill none) (layer "Edge.Cuts"))
 (segment (start 153.698 86.388) (end 152.654 85.344) (width 0.3) (layer "F.Cu") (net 5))
 (segment (start 154.813 86.388) (end 153.698 86.388) (width 0.3) (layer "F.Cu") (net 5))
 (segment (start 144.698 100.229642) (end 144.698 100.813) (width 0.3) (layer "F.Cu") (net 2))
 (segment (start 145.2605 103.237) (end 144.698 102.6745) (width 0.3) (layer "F.Cu") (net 2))
 (segment (start 151.298 92.277) (end 151.298 91.313) (width 0.3) (layer "F.Cu") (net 2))
 (segment (start 151.298 93.629642) (end 144.698 100.229642) (width 0.3) (layer "F.Cu") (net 2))
 (segment (start 152.146 88.392) (end 151.016 88.392) (width 0.3) (layer "F.Cu") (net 2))
 (segment (start 150.863 102.983) (end 149.974 102.094) (width 0.3) (layer "F.Cu") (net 2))
 (segment (start 160.515 99.345) (end 160.279 99.581) (width 0.3) (layer "F.Cu") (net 2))
 (segment (start 152.146 88.392) (end 152.654 88.392) (width 0.3) (layer "F.Cu") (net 2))
 (segment (start 153.498 91.313) (end 153.498 92.213) (width 0.3) (layer "F.Cu") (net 2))
 (segment (start 153.498 92.213) (end 153.148 92.563) (width 0.3) (layer "F.Cu") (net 2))
 (segment (start 161.229 100.531) (end 160.279 99.581) (width 0.3) (layer "F.Cu") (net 2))
 (segment (start 151.298 91.313) (end 151.298 93.629642) (width 0.3) (layer "F.Cu") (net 2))
 (segment (start 149.974 102.094) (end 145.079 102.094) (width 0.3) (layer "F.Cu") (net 2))
 (segment (start 144.698 101.713) (end 144.698 100.813) (width 0.3) (layer "F.Cu") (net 2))
 (segment (start 153.148 92.563) (end 151.584 92.563) (width 0.3) (layer "F.Cu") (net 2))
 (segment (start 145.079 102.094) (end 144.698 101.713) (width 0.3) (layer "F.Cu") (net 2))
 (segment (start 161.229 101.856) (end 161.229 100.531) (width 0.3) (layer "F.Cu") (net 2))
 (segment (start 151.584 92.563) (end 151.298 92.277) (width 0.3) (layer "F.Cu") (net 2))
 (segment (start 144.698 102.6745) (end 144.698 100.813) (width 0.3) (layer "F.Cu") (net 2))
 (segment (start 160.515 97.676) (end 160.515 99.345) (width 0.3) (layer "F.Cu") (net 2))
 (segment (start 152.398 102.968) (end 152.398 100.813) (width 0.3) (layer "F.Cu") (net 4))
 (segment (start 162.179 99.581) (end 162.179 97.79) (width 0.3) (layer "F.Cu") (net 4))
 (segment (start 162.179 97.79) (end 162.065 97.676) (width 0.3) (layer "F.Cu") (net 4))
 (segment (start 152.413 102.983) (end 152.398 102.968) (width 0.3) (layer "F.Cu") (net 4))
 (via (at 153.797 87.122) (size 0.6) (drill 0.3) (layers "F.Cu" "B.Cu") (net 4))
 (segment (start 153.797 87.122) (end 150.762 87.122) (width 0.3) (layer "B.Cu") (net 4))
 (segment (start 154.813 88.288) (end 154.813 87.348) (width 0.3) (layer "F.Cu") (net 16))
 (segment (start 148.205 103.237) (end 146.8355 103.237) (width 0.3) (layer "F.Cu") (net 3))
 (segment (start 154.442 88.392) (end 153.162 88.392) (width 0.3) (layer "F.Cu") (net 17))
 (segment (start 154.813 89.258) (end 154.569 89.014) (width 0.3) (layer "F.Cu") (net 17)))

